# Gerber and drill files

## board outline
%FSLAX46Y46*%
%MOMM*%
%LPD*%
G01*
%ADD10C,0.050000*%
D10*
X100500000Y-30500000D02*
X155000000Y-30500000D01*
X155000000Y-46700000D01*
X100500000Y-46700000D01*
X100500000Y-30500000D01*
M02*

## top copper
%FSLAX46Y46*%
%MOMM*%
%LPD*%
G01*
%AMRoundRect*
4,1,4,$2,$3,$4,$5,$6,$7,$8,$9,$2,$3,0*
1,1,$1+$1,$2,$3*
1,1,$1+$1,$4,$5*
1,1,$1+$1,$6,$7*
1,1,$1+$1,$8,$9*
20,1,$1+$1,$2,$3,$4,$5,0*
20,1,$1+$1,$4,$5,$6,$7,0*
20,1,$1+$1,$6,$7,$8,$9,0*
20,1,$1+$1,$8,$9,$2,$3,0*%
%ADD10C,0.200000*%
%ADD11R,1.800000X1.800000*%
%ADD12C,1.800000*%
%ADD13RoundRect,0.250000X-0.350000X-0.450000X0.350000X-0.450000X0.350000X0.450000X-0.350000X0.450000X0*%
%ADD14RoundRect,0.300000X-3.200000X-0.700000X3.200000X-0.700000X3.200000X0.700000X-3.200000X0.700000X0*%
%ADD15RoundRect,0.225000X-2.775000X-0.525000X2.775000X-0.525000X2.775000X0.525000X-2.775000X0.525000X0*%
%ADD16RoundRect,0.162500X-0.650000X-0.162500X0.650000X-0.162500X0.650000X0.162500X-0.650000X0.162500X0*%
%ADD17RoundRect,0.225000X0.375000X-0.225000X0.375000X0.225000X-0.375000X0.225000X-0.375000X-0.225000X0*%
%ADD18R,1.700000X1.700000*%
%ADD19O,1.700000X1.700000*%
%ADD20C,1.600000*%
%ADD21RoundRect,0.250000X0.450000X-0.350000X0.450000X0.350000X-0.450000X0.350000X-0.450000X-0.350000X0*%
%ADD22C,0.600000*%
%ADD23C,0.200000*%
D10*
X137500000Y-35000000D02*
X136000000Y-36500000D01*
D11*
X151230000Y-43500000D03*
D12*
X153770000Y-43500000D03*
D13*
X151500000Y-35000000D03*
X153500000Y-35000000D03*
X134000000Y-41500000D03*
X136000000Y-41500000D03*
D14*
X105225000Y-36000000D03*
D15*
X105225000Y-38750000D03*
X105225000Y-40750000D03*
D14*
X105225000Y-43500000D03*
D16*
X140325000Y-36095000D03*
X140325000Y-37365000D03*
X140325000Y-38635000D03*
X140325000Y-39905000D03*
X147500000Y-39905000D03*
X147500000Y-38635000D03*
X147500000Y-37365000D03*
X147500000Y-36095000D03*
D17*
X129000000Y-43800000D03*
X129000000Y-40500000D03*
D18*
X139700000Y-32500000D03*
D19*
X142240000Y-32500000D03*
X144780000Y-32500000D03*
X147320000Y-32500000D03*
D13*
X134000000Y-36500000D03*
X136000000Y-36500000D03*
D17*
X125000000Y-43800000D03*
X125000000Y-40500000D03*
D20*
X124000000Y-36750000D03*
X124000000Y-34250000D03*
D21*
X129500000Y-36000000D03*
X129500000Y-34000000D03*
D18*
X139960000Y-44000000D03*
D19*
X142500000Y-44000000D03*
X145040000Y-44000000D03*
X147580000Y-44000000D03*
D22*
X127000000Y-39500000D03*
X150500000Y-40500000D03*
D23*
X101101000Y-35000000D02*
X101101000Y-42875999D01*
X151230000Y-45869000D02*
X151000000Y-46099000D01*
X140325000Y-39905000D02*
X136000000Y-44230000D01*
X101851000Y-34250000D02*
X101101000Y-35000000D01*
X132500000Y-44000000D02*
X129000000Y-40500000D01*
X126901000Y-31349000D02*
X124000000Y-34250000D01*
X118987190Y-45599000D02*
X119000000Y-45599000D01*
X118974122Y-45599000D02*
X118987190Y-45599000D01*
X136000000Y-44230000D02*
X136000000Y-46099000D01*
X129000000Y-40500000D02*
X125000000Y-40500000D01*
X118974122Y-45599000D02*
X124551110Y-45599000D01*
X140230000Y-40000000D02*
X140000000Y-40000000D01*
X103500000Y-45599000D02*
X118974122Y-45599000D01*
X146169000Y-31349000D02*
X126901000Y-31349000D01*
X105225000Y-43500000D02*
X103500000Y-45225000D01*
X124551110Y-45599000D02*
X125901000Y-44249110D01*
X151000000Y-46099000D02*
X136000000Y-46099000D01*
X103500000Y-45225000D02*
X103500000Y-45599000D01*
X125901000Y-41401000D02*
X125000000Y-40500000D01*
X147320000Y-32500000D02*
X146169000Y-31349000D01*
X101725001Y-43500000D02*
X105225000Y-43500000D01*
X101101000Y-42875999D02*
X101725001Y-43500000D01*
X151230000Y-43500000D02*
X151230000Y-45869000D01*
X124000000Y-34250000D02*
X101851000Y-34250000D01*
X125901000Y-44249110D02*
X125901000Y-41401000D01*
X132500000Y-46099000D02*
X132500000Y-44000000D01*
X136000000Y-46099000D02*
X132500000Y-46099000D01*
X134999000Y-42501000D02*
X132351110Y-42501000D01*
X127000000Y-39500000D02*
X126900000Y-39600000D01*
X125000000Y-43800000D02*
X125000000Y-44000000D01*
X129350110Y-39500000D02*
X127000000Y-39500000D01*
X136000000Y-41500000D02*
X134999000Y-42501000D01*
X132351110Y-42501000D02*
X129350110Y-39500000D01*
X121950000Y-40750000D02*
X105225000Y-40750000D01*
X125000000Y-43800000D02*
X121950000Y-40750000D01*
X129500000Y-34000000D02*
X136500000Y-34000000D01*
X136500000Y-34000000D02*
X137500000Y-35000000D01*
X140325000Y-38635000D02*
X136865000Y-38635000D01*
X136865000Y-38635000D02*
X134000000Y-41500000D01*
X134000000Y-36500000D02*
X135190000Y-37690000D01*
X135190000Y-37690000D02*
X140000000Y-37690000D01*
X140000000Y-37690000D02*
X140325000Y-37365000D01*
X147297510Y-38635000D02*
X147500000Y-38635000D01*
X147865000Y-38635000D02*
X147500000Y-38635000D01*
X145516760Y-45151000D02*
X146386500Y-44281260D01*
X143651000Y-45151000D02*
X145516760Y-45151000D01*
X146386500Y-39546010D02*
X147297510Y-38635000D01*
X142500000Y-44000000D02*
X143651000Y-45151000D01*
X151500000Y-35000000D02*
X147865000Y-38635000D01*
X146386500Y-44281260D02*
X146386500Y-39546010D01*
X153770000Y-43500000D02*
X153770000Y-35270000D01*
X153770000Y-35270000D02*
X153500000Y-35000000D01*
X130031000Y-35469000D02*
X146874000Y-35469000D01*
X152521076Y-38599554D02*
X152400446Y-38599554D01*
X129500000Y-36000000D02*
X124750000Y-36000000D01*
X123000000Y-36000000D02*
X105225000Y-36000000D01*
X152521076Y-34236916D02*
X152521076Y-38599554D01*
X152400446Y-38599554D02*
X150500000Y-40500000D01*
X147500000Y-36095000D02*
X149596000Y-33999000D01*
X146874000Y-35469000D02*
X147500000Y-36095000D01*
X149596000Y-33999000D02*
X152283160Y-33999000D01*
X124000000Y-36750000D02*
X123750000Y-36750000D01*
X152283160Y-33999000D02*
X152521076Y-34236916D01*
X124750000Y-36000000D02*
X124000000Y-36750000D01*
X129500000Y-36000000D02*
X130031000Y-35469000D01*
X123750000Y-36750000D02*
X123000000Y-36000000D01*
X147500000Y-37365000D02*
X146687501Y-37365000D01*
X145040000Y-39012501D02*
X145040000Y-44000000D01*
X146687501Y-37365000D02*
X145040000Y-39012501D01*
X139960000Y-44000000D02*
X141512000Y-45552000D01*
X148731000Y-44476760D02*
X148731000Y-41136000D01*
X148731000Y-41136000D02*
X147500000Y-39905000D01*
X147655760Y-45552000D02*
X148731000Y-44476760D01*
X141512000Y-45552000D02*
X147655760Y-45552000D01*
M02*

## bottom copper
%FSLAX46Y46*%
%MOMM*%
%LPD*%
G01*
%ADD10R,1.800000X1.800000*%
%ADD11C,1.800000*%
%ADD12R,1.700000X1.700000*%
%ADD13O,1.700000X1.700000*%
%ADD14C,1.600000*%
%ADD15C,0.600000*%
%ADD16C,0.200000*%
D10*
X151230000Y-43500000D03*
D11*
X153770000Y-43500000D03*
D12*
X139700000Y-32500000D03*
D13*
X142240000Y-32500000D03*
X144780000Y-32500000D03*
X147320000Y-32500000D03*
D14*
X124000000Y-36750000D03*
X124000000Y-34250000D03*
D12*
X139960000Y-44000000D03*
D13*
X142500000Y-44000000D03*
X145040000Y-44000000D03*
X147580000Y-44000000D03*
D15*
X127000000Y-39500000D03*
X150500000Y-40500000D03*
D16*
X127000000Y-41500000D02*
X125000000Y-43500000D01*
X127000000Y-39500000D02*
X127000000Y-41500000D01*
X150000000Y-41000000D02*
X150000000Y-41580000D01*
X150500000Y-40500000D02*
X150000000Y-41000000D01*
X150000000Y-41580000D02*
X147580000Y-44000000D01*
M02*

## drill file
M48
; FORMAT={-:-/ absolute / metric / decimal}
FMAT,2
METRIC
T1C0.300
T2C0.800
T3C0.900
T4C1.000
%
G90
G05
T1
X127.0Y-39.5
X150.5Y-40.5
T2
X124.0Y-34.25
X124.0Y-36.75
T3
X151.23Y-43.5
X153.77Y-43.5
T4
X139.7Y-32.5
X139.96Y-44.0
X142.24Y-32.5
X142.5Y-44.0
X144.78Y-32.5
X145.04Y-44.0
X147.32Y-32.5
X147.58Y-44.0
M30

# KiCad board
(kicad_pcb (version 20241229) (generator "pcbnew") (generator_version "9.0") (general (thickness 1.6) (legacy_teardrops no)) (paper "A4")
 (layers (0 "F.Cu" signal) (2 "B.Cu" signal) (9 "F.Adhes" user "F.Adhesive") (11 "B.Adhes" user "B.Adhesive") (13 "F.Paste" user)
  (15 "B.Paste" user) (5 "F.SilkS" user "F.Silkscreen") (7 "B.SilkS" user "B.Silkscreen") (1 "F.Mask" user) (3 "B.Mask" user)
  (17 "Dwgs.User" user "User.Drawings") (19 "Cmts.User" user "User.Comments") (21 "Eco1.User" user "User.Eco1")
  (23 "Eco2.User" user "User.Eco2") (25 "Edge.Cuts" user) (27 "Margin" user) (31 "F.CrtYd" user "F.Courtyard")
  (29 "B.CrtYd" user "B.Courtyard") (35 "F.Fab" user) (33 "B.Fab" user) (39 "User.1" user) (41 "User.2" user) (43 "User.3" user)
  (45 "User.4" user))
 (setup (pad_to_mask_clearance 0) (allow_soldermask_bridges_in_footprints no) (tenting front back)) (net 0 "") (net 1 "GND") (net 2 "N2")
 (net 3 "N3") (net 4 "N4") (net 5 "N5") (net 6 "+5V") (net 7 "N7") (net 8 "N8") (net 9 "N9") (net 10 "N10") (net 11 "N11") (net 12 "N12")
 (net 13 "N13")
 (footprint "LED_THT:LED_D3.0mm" (layer "F.Cu") (at 151.23 43.5)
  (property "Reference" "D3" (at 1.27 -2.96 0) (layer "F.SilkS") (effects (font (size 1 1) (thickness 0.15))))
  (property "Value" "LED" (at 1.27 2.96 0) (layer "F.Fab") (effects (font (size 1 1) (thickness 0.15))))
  (pad "1" thru_hole rect (at 0 0) (size 1.8 1.8) (drill 0.9) (layers "*.Cu" "*.Mask") (remove_unused_layers no) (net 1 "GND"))
  (pad "2" thru_hole circle (at 2.54 0) (size 1.8 1.8) (drill 0.9) (layers "*.Cu" "*.Mask") (remove_unused_layers no) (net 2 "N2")))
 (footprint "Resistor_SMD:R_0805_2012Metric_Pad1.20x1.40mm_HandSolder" (layer "F.Cu") (at 152.5 35)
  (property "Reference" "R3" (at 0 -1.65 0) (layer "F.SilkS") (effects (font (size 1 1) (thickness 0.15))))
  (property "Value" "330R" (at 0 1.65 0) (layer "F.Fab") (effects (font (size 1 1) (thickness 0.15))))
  (pad "1" smd roundrect (at -1 0) (size 1.2 1.4) (layers "F.Cu" "F.Mask" "F.Paste") (roundrect_rratio 0.208333) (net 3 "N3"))
  (pad "2" smd roundrect (at 1 0) (size 1.2 1.4) (layers "F.Cu" "F.Mask" "F.Paste") (roundrect_rratio 0.208333) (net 2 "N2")))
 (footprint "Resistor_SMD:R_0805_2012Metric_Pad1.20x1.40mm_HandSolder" (layer "F.Cu") (at 135 41.5)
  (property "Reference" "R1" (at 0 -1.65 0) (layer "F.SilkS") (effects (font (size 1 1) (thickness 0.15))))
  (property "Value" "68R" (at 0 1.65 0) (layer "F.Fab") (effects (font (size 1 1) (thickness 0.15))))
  (pad "1" smd roundrect (at -1 0) (size 1.2 1.4) (layers "F.Cu" "F.Mask" "F.Paste") (roundrect_rratio 0.208333) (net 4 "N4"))
  (pad "2" smd roundrect (at 1 0) (size 1.2 1.4) (layers "F.Cu" "F.Mask" "F.Paste") (roundrect_rratio 0.208333) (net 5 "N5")))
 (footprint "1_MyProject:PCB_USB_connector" (layer "F.Cu") (at 105.225 39.75)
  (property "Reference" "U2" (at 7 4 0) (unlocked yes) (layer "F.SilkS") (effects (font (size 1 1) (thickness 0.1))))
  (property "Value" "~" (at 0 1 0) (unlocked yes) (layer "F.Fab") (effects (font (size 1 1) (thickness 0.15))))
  (pad "1" smd roundrect (at 0 -3.75) (size 7 2) (layers "F.Cu" "F.Mask" "F.Paste") (roundrect_rratio 0.15) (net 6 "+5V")
   (thermal_bridge_angle 45))
  (pad "2" smd roundrect (at 0 -1) (size 6 1.5) (layers "F.Cu" "F.Mask" "F.Paste") (roundrect_rratio 0.15) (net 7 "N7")
   (thermal_bridge_angle 45))
  (pad "3" smd roundrect (at 0 1) (size 6 1.5) (layers "F.Cu" "F.Mask" "F.Paste") (roundrect_rratio 0.15) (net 5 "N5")
   (thermal_bridge_angle 45))
  (pad "4" smd roundrect (at 0 3.75) (size 7 2) (layers "F.Cu" "F.Mask" "F.Paste") (roundrect_rratio 0.15) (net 1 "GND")
   (thermal_bridge_angle 45)))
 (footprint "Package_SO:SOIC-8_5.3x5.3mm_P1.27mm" (layer "F.Cu") (at 143.9125 38)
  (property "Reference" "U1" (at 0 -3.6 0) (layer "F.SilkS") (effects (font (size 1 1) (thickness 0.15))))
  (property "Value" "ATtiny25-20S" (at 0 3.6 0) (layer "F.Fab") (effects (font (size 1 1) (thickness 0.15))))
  (pad "1" smd roundrect (at -3.5875 -1.905) (size 1.625 0.65) (layers "F.Cu" "F.Mask" "F.Paste") (roundrect_rratio 0.25) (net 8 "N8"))
  (pad "2" smd roundrect (at -3.5875 -0.635) (size 1.625 0.65) (layers "F.Cu" "F.Mask" "F.Paste") (roundrect_rratio 0.25) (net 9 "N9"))
  (pad "3" smd roundrect (at -3.5875 0.635) (size 1.625 0.65) (layers "F.Cu" "F.Mask" "F.Paste") (roundrect_rratio 0.25) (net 4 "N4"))
  (pad "4" smd roundrect (at -3.5875 1.905) (size 1.625 0.65) (layers "F.Cu" "F.Mask" "F.Paste") (roundrect_rratio 0.25) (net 1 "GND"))
  (pad "5" smd roundrect (at 3.5875 1.905) (size 1.625 0.65) (layers "F.Cu" "F.Mask" "F.Paste") (roundrect_rratio 0.25) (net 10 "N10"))
  (pad "6" smd roundrect (at 3.5875 0.635) (size 1.625 0.65) (layers "F.Cu" "F.Mask" "F.Paste") (roundrect_rratio 0.25) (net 3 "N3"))
  (pad "7" smd roundrect (at 3.5875 -0.635) (size 1.625 0.65) (layers "F.Cu" "F.Mask" "F.Paste") (roundrect_rratio 0.25) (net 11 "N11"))
  (pad "8" smd roundrect (at 3.5875 -1.905) (size 1.625 0.65) (layers "F.Cu" "F.Mask" "F.Paste") (roundrect_rratio 0.25) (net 6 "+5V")))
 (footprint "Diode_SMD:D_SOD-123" (layer "F.Cu") (at 129 42.15 90)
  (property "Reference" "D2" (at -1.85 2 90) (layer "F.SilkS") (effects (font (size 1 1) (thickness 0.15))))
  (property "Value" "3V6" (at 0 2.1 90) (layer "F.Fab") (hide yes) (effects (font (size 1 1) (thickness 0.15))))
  (pad "1" smd roundrect (at -1.65 0 90) (size 0.9 1.2) (layers "F.Cu" "F.Mask" "F.Paste") (roundrect_rratio 0.25) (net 7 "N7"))
  (pad "2" smd roundrect (at 1.65 0 90) (size 0.9 1.2) (layers "F.Cu" "F.Mask" "F.Paste") (roundrect_rratio 0.25) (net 1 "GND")))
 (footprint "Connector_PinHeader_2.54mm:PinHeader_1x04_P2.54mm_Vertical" (layer "F.Cu") (at 139.7 32.5 90)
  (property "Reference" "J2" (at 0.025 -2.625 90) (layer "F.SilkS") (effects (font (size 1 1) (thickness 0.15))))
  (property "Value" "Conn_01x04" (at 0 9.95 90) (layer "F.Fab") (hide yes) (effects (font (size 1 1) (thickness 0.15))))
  (pad "1" thru_hole rect (at 0 0 90) (size 1.7 1.7) (drill 1) (layers "*.Cu" "*.Mask") (remove_unused_layers no) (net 8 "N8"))
  (pad "2" thru_hole oval (at 0 2.54 90) (size 1.7 1.7) (drill 1) (layers "*.Cu" "*.Mask") (remove_unused_layers no) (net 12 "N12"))
  (pad "3" thru_hole oval (at 0 5.08 90) (size 1.7 1.7) (drill 1) (layers "*.Cu" "*.Mask") (remove_unused_layers no) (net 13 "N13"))
  (pad "4" thru_hole oval (at 0 7.62 90) (size 1.7 1.7) (drill 1) (layers "*.Cu" "*.Mask") (remove_unused_layers no) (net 1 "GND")))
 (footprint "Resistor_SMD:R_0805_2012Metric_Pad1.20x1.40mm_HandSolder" (layer "F.Cu") (at 135 36.5)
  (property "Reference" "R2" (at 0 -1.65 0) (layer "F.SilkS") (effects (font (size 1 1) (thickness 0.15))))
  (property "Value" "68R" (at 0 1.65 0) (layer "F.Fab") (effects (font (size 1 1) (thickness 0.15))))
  (pad "1" smd roundrect (at -1 0) (size 1.2 1.4) (layers "F.Cu" "F.Mask" "F.Paste") (roundrect_rratio 0.208333) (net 9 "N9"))
  (pad "2" smd roundrect (at 1 0) (size 1.2 1.4) (layers "F.Cu" "F.Mask" "F.Paste") (roundrect_rratio 0.208333) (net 7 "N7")))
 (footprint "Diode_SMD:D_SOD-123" (layer "F.Cu") (at 125 42.15 90)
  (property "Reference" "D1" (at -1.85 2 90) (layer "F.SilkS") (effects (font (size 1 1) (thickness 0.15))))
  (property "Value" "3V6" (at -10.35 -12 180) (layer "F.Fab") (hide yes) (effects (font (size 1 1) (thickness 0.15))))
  (pad "1" smd roundrect (at -1.65 0 90) (size 0.9 1.2) (layers "F.Cu" "F.Mask" "F.Paste") (roundrect_rratio 0.25) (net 5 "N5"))
  (pad "2" smd roundrect (at 1.65 0 90) (size 0.9 1.2) (layers "F.Cu" "F.Mask" "F.Paste") (roundrect_rratio 0.25) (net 1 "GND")))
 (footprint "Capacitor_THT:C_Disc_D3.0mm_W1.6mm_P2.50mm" (layer "F.Cu") (at 124 36.75 90)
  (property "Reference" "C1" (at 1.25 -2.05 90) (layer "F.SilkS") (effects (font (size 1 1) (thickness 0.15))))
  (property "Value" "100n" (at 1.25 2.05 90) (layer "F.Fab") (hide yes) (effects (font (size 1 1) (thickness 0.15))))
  (pad "1" thru_hole circle (at 0 0 90) (size 1.6 1.6) (drill 0.8) (layers "*.Cu" "*.Mask") (remove_unused_layers no) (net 6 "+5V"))
  (pad "2" thru_hole circle (at 2.5 0 90) (size 1.6 1.6) (drill 0.8) (layers "*.Cu" "*.Mask") (remove_unused_layers no) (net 1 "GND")))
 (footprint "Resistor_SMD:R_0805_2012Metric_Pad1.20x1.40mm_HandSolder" (layer "F.Cu") (at 129.5 35 90)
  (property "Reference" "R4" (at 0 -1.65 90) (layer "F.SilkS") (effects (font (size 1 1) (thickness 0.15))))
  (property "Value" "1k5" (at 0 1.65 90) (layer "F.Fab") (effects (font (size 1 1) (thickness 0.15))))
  (pad "1" smd roundrect (at -1 0 90) (size 1.2 1.4) (layers "F.Cu" "F.Mask" "F.Paste") (roundrect_rratio 0.208333) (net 6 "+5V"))
  (pad "2" smd roundrect (at 1 0 90) (size 1.2 1.4) (layers "F.Cu" "F.Mask" "F.Paste") (roundrect_rratio 0.208333) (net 7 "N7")))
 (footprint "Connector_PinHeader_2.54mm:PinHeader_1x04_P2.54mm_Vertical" (layer "F.Cu") (at 139.96 44 90)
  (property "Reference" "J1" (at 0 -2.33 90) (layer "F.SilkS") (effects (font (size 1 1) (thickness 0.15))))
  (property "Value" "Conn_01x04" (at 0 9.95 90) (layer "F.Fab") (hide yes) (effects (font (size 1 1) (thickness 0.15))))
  (pad "1" thru_hole rect (at 0 0 90) (size 1.7 1.7) (drill 1) (layers "*.Cu" "*.Mask") (remove_unused_layers no) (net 10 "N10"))
  (pad "2" thru_hole oval (at 0 2.54 90) (size 1.7 1.7) (drill 1) (layers "*.Cu" "*.Mask") (remove_unused_layers no) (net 3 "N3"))
  (pad "3" thru_hole oval (at 0 5.08 90) (size 1.7 1.7) (drill 1) (layers "*.Cu" "*.Mask") (remove_unused_layers no) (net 11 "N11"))
  (pad "4" thru_hole oval (at 0 7.62 90) (size 1.7 1.7) (drill 1) (layers "*.Cu" "*.Mask") (remove_unused_layers no) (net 6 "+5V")))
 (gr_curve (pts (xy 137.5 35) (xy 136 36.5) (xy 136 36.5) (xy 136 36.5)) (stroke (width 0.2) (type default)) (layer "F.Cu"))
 (gr_rect (start 100.5 30.5) (end 155 46.7) (stroke (width 0.05) (type solid)) (fill no) (layer "Edge.Cuts"))
 (segment (start 101.101 35) (end 101.101 42.875999) (width 0.2) (layer "F.Cu") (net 1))
 (segment (start 151.23 45.869) (end 151 46.099) (width 0.2) (layer "F.Cu") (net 1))
 (segment (start 140.325 39.905) (end 136 44.23) (width 0.2) (layer "F.Cu") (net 1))
 (segment (start 101.851 34.25) (end 101.101 35) (width 0.2) (layer "F.Cu") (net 1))
 (segment (start 132.5 44) (end 129 40.5) (width 0.2) (layer "F.Cu") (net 1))
 (segment (start 126.901 31.349) (end 124 34.25) (width 0.2) (layer "F.Cu") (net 1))
 (segment (start 118.98719 45.599) (end 119 45.599) (width 0.2) (layer "F.Cu") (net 1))
 (segment (start 118.974122 45.599) (end 118.98719 45.599) (width 0.2) (layer "F.Cu") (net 1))
 (segment (start 136 44.23) (end 136 46.099) (width 0.2) (layer "F.Cu") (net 1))
 (segment (start 129 40.5) (end 125 40.5) (width 0.2) (layer "F.Cu") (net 1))
 (segment (start 118.974122 45.599) (end 124.55111 45.599) (width 0.2) (layer "F.Cu") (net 1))
 (segment (start 140.23 40) (end 140 40) (width 0.2) (layer "F.Cu") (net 1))
 (segment (start 103.5 45.599) (end 118.974122 45.599) (width 0.2) (layer "F.Cu") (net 1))
 (segment (start 146.169 31.349) (end 126.901 31.349) (width 0.2) (layer "F.Cu") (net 1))
 (segment (start 105.225 43.5) (end 103.5 45.225) (width 0.2) (layer "F.Cu") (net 1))
 (segment (start 124.55111 45.599) (end 125.901 44.24911) (width 0.2) (layer "F.Cu") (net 1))
 (segment (start 151 46.099) (end 136 46.099) (width 0.2) (layer "F.Cu") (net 1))
 (segment (start 103.5 45.225) (end 103.5 45.599) (width 0.2) (layer "F.Cu") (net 1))
 (segment (start 125.901 41.401) (end 125 40.5) (width 0.2) (layer "F.Cu") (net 1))
 (segment (start 147.32 32.5) (end 146.169 31.349) (width 0.2) (layer "F.Cu") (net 1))
 (segment (start 101.725001 43.5) (end 105.225 43.5) (width 0.2) (layer "F.Cu") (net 1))
 (segment (start 101.101 42.875999) (end 101.725001 43.5) (width 0.2) (layer "F.Cu") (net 1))
 (segment (start 151.23 43.5) (end 151.23 45.869) (width 0.2) (layer "F.Cu") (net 1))
 (segment (start 124 34.25) (end 101.851 34.25) (width 0.2) (layer "F.Cu") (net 1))
 (segment (start 125.901 44.24911) (end 125.901 41.401) (width 0.2) (layer "F.Cu") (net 1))
 (segment (start 132.5 46.099) (end 132.5 44) (width 0.2) (layer "F.Cu") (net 1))
 (segment (start 136 46.099) (end 132.5 46.099) (width 0.2) (layer "F.Cu") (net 1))
 (segment (start 134.999 42.501) (end 132.35111 42.501) (width 0.2) (layer "F.Cu") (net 5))
 (segment (start 127 39.5) (end 126.9 39.6) (width 0.2) (layer "F.Cu") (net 5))
 (segment (start 125 43.8) (end 125 44) (width 0.2) (layer "F.Cu") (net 5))
 (segment (start 129.35011 39.5) (end 127 39.5) (width 0.2) (layer "F.Cu") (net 5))
 (segment (start 136 41.5) (end 134.999 42.501) (width 0.2) (layer "F.Cu") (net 5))
 (segment (start 132.35111 42.501) (end 129.35011 39.5) (width 0.2) (layer "F.Cu") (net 5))
 (segment (start 121.95 40.75) (end 105.225 40.75) (width 0.2) (layer "F.Cu") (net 5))
 (segment (start 125 43.8) (end 121.95 40.75) (width 0.2) (layer "F.Cu") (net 5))
 (via (at 127 39.5) (size 0.6) (drill 0.3) (layers "F.Cu" "B.Cu") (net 5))
 (segment (start 127 41.5) (end 125 43.5) (width 0.2) (layer "B.Cu") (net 5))
 (segment (start 127 39.5) (end 127 41.5) (width 0.2) (layer "B.Cu") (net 5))
 (segment (start 129.5 34) (end 136.5 34) (width 0.2) (layer "F.Cu") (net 7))
 (segment (start 136.5 34) (end 137.5 35) (width 0.2) (layer "F.Cu") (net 7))
 (segment (start 140.325 38.635) (end 136.865 38.635) (width 0.2) (layer "F.Cu") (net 4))
 (segment (start 136.865 38.635) (end 134 41.5) (width 0.2) (layer "F.Cu") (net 4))
 (segment (start 134 36.5) (end 135.19 37.69) (width 0.2) (layer "F.Cu") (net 9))
 (segment (start 135.19 37.69) (end 140 37.69) (width 0.2) (layer "F.Cu") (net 9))
 (segment (start 140 37.69) (end 140.325 37.365) (width 0.2) (layer "F.Cu") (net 9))
 (segment (start 147.29751 38.635) (end 147.5 38.635) (width 0.2) (layer "F.Cu") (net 3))
 (segment (start 147.865 38.635) (end 147.5 38.635) (width 0.2) (layer "F.Cu") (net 3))
 (segment (start 145.51676 45.151) (end 146.3865 44.28126) (width 0.2) (layer "F.Cu") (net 3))
 (segment (start 143.651 45.151) (end 145.51676 45.151) (width 0.2) (layer "F.Cu") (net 3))
 (segment (start 146.3865 39.54601) (end 147.29751 38.635) (width 0.2) (layer "F.Cu") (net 3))
 (segment (start 142.5 44) (end 143.651 45.151) (width 0.2) (layer "F.Cu") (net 3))
 (segment (start 151.5 35) (end 147.865 38.635) (width 0.2) (layer "F.Cu") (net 3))
 (segment (start 146.3865 44.28126) (end 146.3865 39.54601) (width 0.2) (layer "F.Cu") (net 3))
 (segment (start 153.77 43.5) (end 153.77 35.27) (width 0.2) (layer "F.Cu") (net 2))
 (segment (start 153.77 35.27) (end 153.5 35) (width 0.2) (layer "F.Cu") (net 2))
 (segment (start 130.031 35.469) (end 146.874 35.469) (width 0.2) (layer "F.Cu") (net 6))
 (segment (start 152.521076 38.599554) (end 152.400446 38.599554) (width 0.2) (layer "F.Cu") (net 6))
 (segment (start 129.5 36) (end 124.75 36) (width 0.2) (layer "F.Cu") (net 6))
 (segment (start 123 36) (end 105.225 36) (width 0.2) (layer "F.Cu") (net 6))
 (segment (start 152.521076 34.236916) (end 152.521076 38.599554) (width 0.2) (layer "F.Cu") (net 6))
 (segment (start 152.400446 38.599554) (end 150.5 40.5) (width 0.2) (layer "F.Cu") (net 6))
 (segment (start 147.5 36.095) (end 149.596 33.999) (width 0.2) (layer "F.Cu") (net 6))
 (segment (start 146.874 35.469) (end 147.5 36.095) (width 0.2) (layer "F.Cu") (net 6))
 (segment (start 149.596 33.999) (end 152.28316 33.999) (width 0.2) (layer "F.Cu") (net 6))
 (segment (start 124 36.75) (end 123.75 36.75) (width 0.2) (layer "F.Cu") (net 6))
 (segment (start 152.28316 33.999) (end 152.521076 34.236916) (width 0.2) (layer "F.Cu") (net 6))
 (segment (start 124.75 36) (end 124 36.75) (width 0.2) (layer "F.Cu") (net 6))
 (segment (start 129.5 36) (end 130.031 35.469) (width 0.2) (layer "F.Cu") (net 6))
 (segment (start 123.75 36.75) (end 123 36) (width 0.2) (layer "F.Cu") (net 6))
 (via (at 150.5 40.5) (size 0.6) (drill 0.3) (layers "F.Cu" "B.Cu") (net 6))
 (segment (start 150 41) (end 150 41.58) (width 0.2) (layer "B.Cu") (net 6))
 (segment (start 150.5 40.5) (end 150 41) (width 0.2) (layer "B.Cu") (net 6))
 (segment (start 150 41.58) (end 147.58 44) (width 0.2) (layer "B.Cu") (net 6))
 (segment (start 147.5 37.365) (end 146.687501 37.365) (width 0.2) (layer "F.Cu") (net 11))
 (segment (start 145.04 39.012501) (end 145.04 44) (width 0.2) (layer "F.Cu") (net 11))
 (segment (start 146.687501 37.365) (end 145.04 39.012501) (width 0.2) (layer "F.Cu") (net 11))
 (segment (start 139.96 44) (end 141.512 45.552) (width 0.2) (layer "F.Cu") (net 10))
 (segment (start 148.731 44.47676) (end 148.731 41.136) (width 0.2) (layer "F.Cu") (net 10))
 (segment (start 148.731 41.136) (end 147.5 39.905) (width 0.2) (layer "F.Cu") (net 10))
 (segment (start 147.65576 45.552) (end 148.731 44.47676) (width 0.2) (layer "F.Cu") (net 10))
 (segment (start 141.512 45.552) (end 147.65576 45.552) (width 0.2) (layer "F.Cu") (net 10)))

